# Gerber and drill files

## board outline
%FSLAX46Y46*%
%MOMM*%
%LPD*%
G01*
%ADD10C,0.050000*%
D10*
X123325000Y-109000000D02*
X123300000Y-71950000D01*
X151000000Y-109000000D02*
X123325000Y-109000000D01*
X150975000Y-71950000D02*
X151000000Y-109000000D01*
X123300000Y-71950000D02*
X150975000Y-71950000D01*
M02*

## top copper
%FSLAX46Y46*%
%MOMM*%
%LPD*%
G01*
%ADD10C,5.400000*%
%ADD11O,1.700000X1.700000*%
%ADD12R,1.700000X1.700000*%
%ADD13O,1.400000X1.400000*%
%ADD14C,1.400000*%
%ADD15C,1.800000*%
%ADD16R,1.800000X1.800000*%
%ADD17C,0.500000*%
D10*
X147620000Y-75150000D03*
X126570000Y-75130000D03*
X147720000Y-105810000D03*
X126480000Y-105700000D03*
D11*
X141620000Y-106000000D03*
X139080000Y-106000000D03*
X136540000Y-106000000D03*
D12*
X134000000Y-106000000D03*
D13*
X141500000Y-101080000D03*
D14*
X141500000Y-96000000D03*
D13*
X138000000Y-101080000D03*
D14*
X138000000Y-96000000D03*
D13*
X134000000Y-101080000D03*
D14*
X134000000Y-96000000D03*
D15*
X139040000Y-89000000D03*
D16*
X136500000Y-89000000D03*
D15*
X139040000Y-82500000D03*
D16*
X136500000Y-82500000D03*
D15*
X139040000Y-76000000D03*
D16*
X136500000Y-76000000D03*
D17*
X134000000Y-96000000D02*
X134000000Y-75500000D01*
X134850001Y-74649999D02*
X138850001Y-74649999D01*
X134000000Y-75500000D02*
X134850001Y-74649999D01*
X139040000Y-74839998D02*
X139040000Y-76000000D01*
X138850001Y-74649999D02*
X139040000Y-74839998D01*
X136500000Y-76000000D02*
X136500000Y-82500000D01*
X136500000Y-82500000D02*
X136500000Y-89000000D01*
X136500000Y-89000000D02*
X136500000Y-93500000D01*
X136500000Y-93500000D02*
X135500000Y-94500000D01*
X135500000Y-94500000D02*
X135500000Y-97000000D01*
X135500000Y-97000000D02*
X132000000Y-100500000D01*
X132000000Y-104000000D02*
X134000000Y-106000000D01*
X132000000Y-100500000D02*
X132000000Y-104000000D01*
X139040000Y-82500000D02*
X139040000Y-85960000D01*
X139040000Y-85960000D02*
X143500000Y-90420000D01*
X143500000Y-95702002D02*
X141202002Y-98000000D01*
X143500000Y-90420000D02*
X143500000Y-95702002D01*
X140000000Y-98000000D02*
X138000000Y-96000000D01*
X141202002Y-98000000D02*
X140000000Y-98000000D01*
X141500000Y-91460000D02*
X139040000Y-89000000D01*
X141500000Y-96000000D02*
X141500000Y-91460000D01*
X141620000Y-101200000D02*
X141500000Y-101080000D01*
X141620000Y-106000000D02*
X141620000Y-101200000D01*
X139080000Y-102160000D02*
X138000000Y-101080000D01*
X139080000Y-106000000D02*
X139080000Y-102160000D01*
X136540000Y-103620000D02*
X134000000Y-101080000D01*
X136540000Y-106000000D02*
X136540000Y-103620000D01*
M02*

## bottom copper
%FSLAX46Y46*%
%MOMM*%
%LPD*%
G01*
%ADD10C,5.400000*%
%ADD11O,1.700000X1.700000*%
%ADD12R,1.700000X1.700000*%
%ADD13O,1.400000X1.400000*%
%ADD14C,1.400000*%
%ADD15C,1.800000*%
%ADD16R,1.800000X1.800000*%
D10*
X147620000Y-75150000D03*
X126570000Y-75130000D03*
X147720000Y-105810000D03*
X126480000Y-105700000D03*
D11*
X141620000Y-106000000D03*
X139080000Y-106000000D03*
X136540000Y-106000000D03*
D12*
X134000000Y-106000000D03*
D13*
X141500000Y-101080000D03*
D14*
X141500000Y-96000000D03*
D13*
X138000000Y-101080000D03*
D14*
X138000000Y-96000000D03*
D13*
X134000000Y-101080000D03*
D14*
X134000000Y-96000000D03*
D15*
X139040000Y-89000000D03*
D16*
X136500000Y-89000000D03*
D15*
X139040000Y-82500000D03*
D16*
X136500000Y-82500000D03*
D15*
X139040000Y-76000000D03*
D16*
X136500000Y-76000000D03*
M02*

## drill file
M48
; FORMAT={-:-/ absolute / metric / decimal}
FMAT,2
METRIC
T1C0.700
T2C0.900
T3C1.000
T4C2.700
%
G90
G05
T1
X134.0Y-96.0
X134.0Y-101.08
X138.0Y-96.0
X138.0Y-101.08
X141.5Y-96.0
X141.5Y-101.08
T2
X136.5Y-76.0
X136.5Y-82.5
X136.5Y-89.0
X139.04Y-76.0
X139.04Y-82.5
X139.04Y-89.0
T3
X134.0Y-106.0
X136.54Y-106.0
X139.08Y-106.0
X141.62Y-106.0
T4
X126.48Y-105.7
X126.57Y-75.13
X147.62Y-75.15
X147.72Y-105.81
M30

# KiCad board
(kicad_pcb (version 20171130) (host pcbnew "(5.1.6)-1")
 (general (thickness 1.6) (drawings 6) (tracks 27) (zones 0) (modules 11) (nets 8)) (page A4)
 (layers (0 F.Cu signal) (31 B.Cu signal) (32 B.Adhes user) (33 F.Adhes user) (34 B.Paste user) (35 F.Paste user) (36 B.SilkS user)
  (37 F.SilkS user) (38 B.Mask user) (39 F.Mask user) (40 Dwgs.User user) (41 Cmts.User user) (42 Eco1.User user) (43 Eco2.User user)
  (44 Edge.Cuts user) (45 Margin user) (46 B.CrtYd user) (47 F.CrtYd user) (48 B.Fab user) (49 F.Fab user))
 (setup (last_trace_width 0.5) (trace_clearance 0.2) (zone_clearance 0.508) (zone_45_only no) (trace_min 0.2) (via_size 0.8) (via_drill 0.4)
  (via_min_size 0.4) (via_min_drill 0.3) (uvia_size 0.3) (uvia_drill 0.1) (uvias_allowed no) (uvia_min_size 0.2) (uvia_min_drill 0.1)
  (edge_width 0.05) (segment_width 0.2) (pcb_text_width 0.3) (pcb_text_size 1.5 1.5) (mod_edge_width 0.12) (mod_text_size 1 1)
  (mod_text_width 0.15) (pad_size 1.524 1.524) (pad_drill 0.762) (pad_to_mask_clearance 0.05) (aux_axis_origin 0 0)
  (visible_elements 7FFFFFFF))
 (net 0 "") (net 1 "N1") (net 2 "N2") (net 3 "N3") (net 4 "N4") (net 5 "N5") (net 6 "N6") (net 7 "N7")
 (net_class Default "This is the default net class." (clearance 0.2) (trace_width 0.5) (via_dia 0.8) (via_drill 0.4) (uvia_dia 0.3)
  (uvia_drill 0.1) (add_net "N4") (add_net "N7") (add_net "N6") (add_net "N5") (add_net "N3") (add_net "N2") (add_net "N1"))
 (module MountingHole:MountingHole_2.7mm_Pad (layer F.Cu) (at 147.62 75.15)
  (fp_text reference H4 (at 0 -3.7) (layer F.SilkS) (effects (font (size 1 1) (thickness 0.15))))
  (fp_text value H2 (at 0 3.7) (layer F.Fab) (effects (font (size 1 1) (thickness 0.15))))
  (pad 1 thru_hole circle (at 0 0) (size 5.4 5.4) (drill 2.7) (layers *.Cu *.Mask)))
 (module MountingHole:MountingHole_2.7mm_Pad (layer F.Cu) (at 126.57 75.13)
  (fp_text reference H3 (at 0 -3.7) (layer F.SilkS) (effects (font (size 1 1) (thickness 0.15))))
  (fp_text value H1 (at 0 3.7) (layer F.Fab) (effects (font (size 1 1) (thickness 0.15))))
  (pad 1 thru_hole circle (at 0 0) (size 5.4 5.4) (drill 2.7) (layers *.Cu *.Mask)))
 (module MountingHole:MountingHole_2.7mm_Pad (layer F.Cu) (at 147.72 105.81)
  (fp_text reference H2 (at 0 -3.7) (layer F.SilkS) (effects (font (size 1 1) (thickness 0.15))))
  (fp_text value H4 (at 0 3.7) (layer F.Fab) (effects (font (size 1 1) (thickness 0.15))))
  (pad 1 thru_hole circle (at 0 0) (size 5.4 5.4) (drill 2.7) (layers *.Cu *.Mask)))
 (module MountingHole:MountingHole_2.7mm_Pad (layer F.Cu) (at 126.48 105.7)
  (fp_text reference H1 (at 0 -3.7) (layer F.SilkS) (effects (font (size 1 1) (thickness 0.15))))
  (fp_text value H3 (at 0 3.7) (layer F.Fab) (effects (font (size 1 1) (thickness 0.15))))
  (pad 1 thru_hole circle (at 0 0) (size 5.4 5.4) (drill 2.7) (layers *.Cu *.Mask)))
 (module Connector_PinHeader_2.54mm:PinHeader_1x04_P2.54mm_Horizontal (layer B.Cu) (at 134 106 270)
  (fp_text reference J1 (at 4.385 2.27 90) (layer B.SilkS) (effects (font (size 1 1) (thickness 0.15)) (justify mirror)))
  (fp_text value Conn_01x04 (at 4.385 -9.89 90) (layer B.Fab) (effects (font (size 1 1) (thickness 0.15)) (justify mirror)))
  (pad 4 thru_hole oval (at 0 -7.62 270) (size 1.7 1.7) (drill 1) (layers *.Cu *.Mask) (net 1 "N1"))
  (pad 3 thru_hole oval (at 0 -5.08 270) (size 1.7 1.7) (drill 1) (layers *.Cu *.Mask) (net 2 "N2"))
  (pad 2 thru_hole oval (at 0 -2.54 270) (size 1.7 1.7) (drill 1) (layers *.Cu *.Mask) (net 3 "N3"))
  (pad 1 thru_hole rect (at 0 0 270) (size 1.7 1.7) (drill 1) (layers *.Cu *.Mask) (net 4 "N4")))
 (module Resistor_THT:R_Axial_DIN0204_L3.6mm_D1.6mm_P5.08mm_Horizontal (layer F.Cu) (at 141.5 96 270)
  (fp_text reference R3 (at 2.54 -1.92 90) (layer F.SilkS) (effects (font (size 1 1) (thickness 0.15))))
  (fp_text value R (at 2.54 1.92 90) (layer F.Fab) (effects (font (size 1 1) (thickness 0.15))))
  (pad 2 thru_hole oval (at 5.08 0 270) (size 1.4 1.4) (drill 0.7) (layers *.Cu *.Mask) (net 1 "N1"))
  (pad 1 thru_hole circle (at 0 0 270) (size 1.4 1.4) (drill 0.7) (layers *.Cu *.Mask) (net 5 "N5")))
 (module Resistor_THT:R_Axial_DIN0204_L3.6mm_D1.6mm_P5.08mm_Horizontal (layer F.Cu) (at 138 96 270)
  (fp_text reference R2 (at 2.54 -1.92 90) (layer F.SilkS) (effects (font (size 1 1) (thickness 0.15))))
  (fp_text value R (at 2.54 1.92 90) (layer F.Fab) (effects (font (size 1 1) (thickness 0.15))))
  (pad 2 thru_hole oval (at 5.08 0 270) (size 1.4 1.4) (drill 0.7) (layers *.Cu *.Mask) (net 2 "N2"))
  (pad 1 thru_hole circle (at 0 0 270) (size 1.4 1.4) (drill 0.7) (layers *.Cu *.Mask) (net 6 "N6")))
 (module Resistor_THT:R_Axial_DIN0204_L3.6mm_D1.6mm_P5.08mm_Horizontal (layer F.Cu) (at 134 96 270)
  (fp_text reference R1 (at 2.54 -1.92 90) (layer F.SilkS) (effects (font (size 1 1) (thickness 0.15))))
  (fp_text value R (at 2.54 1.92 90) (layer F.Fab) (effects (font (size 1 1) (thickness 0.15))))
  (pad 2 thru_hole oval (at 5.08 0 270) (size 1.4 1.4) (drill 0.7) (layers *.Cu *.Mask) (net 3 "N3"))
  (pad 1 thru_hole circle (at 0 0 270) (size 1.4 1.4) (drill 0.7) (layers *.Cu *.Mask) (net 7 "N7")))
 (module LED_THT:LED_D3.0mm (layer F.Cu) (at 136.5 89)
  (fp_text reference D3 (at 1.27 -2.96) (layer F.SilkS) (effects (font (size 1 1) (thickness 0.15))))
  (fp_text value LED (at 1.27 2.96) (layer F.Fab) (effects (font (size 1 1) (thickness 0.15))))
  (pad 2 thru_hole circle (at 2.54 0) (size 1.8 1.8) (drill 0.9) (layers *.Cu *.Mask) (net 5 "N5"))
  (pad 1 thru_hole rect (at 0 0) (size 1.8 1.8) (drill 0.9) (layers *.Cu *.Mask) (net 4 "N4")))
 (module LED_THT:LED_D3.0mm (layer F.Cu) (at 136.5 82.5)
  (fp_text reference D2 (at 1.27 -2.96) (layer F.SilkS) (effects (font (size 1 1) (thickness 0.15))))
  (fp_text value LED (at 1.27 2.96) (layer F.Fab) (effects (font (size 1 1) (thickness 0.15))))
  (pad 2 thru_hole circle (at 2.54 0) (size 1.8 1.8) (drill 0.9) (layers *.Cu *.Mask) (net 6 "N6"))
  (pad 1 thru_hole rect (at 0 0) (size 1.8 1.8) (drill 0.9) (layers *.Cu *.Mask) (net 4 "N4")))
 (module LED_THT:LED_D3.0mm (layer F.Cu) (at 136.5 76)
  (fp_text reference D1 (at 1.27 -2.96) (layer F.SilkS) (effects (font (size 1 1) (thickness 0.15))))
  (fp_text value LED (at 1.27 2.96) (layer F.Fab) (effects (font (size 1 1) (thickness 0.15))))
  (pad 2 thru_hole circle (at 2.54 0) (size 1.8 1.8) (drill 0.9) (layers *.Cu *.Mask) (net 7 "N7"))
  (pad 1 thru_hole rect (at 0 0) (size 1.8 1.8) (drill 0.9) (layers *.Cu *.Mask) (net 4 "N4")))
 (gr_line (start 123.325 109) (end 123.3 71.95) (layer Edge.Cuts) (width 0.05))
 (gr_line (start 151 109) (end 123.325 109) (layer Edge.Cuts) (width 0.05))
 (gr_line (start 150.975 71.95) (end 151 109) (layer Edge.Cuts) (width 0.05))
 (gr_line (start 123.3 71.95) (end 150.975 71.95) (layer Edge.Cuts) (width 0.05))
 (segment (start 134 96) (end 134 75.5) (width 0.5) (layer F.Cu) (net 7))
 (segment (start 134.850001 74.649999) (end 138.850001 74.649999) (width 0.5) (layer F.Cu) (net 7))
 (segment (start 134 75.5) (end 134.850001 74.649999) (width 0.5) (layer F.Cu) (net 7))
 (segment (start 139.04 74.839998) (end 139.04 76) (width 0.5) (layer F.Cu) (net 7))
 (segment (start 138.850001 74.649999) (end 139.04 74.839998) (width 0.5) (layer F.Cu) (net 7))
 (segment (start 136.5 76) (end 136.5 82.5) (width 0.5) (layer F.Cu) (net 4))
 (segment (start 136.5 82.5) (end 136.5 89) (width 0.5) (layer F.Cu) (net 4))
 (segment (start 136.5 89) (end 136.5 93.5) (width 0.5) (layer F.Cu) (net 4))
 (segment (start 136.5 93.5) (end 135.5 94.5) (width 0.5) (layer F.Cu) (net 4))
 (segment (start 135.5 94.5) (end 135.5 97) (width 0.5) (layer F.Cu) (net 4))
 (segment (start 135.5 97) (end 132 100.5) (width 0.5) (layer F.Cu) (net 4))
 (segment (start 132 104) (end 134 106) (width 0.5) (layer F.Cu) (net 4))
 (segment (start 132 100.5) (end 132 104) (width 0.5) (layer F.Cu) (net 4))
 (segment (start 139.04 82.5) (end 139.04 85.96) (width 0.5) (layer F.Cu) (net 6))
 (segment (start 139.04 85.96) (end 143.5 90.42) (width 0.5) (layer F.Cu) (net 6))
 (segment (start 143.5 95.702002) (end 141.202002 98) (width 0.5) (layer F.Cu) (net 6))
 (segment (start 143.5 90.42) (end 143.5 95.702002) (width 0.5) (layer F.Cu) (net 6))
 (segment (start 140 98) (end 138 96) (width 0.5) (layer F.Cu) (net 6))
 (segment (start 141.202002 98) (end 140 98) (width 0.5) (layer F.Cu) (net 6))
 (segment (start 141.5 91.46) (end 139.04 89) (width 0.5) (layer F.Cu) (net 5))
 (segment (start 141.5 96) (end 141.5 91.46) (width 0.5) (layer F.Cu) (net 5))
 (segment (start 141.62 101.2) (end 141.5 101.08) (width 0.5) (layer F.Cu) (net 1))
 (segment (start 141.62 106) (end 141.62 101.2) (width 0.5) (layer F.Cu) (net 1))
 (segment (start 139.08 102.16) (end 138 101.08) (width 0.5) (layer F.Cu) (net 2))
 (segment (start 139.08 106) (end 139.08 102.16) (width 0.5) (layer F.Cu) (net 2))
 (segment (start 136.54 103.62) (end 134 101.08) (width 0.5) (layer F.Cu) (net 3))
 (segment (start 136.54 106) (end 136.54 103.62) (width 0.5) (layer F.Cu) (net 3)))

